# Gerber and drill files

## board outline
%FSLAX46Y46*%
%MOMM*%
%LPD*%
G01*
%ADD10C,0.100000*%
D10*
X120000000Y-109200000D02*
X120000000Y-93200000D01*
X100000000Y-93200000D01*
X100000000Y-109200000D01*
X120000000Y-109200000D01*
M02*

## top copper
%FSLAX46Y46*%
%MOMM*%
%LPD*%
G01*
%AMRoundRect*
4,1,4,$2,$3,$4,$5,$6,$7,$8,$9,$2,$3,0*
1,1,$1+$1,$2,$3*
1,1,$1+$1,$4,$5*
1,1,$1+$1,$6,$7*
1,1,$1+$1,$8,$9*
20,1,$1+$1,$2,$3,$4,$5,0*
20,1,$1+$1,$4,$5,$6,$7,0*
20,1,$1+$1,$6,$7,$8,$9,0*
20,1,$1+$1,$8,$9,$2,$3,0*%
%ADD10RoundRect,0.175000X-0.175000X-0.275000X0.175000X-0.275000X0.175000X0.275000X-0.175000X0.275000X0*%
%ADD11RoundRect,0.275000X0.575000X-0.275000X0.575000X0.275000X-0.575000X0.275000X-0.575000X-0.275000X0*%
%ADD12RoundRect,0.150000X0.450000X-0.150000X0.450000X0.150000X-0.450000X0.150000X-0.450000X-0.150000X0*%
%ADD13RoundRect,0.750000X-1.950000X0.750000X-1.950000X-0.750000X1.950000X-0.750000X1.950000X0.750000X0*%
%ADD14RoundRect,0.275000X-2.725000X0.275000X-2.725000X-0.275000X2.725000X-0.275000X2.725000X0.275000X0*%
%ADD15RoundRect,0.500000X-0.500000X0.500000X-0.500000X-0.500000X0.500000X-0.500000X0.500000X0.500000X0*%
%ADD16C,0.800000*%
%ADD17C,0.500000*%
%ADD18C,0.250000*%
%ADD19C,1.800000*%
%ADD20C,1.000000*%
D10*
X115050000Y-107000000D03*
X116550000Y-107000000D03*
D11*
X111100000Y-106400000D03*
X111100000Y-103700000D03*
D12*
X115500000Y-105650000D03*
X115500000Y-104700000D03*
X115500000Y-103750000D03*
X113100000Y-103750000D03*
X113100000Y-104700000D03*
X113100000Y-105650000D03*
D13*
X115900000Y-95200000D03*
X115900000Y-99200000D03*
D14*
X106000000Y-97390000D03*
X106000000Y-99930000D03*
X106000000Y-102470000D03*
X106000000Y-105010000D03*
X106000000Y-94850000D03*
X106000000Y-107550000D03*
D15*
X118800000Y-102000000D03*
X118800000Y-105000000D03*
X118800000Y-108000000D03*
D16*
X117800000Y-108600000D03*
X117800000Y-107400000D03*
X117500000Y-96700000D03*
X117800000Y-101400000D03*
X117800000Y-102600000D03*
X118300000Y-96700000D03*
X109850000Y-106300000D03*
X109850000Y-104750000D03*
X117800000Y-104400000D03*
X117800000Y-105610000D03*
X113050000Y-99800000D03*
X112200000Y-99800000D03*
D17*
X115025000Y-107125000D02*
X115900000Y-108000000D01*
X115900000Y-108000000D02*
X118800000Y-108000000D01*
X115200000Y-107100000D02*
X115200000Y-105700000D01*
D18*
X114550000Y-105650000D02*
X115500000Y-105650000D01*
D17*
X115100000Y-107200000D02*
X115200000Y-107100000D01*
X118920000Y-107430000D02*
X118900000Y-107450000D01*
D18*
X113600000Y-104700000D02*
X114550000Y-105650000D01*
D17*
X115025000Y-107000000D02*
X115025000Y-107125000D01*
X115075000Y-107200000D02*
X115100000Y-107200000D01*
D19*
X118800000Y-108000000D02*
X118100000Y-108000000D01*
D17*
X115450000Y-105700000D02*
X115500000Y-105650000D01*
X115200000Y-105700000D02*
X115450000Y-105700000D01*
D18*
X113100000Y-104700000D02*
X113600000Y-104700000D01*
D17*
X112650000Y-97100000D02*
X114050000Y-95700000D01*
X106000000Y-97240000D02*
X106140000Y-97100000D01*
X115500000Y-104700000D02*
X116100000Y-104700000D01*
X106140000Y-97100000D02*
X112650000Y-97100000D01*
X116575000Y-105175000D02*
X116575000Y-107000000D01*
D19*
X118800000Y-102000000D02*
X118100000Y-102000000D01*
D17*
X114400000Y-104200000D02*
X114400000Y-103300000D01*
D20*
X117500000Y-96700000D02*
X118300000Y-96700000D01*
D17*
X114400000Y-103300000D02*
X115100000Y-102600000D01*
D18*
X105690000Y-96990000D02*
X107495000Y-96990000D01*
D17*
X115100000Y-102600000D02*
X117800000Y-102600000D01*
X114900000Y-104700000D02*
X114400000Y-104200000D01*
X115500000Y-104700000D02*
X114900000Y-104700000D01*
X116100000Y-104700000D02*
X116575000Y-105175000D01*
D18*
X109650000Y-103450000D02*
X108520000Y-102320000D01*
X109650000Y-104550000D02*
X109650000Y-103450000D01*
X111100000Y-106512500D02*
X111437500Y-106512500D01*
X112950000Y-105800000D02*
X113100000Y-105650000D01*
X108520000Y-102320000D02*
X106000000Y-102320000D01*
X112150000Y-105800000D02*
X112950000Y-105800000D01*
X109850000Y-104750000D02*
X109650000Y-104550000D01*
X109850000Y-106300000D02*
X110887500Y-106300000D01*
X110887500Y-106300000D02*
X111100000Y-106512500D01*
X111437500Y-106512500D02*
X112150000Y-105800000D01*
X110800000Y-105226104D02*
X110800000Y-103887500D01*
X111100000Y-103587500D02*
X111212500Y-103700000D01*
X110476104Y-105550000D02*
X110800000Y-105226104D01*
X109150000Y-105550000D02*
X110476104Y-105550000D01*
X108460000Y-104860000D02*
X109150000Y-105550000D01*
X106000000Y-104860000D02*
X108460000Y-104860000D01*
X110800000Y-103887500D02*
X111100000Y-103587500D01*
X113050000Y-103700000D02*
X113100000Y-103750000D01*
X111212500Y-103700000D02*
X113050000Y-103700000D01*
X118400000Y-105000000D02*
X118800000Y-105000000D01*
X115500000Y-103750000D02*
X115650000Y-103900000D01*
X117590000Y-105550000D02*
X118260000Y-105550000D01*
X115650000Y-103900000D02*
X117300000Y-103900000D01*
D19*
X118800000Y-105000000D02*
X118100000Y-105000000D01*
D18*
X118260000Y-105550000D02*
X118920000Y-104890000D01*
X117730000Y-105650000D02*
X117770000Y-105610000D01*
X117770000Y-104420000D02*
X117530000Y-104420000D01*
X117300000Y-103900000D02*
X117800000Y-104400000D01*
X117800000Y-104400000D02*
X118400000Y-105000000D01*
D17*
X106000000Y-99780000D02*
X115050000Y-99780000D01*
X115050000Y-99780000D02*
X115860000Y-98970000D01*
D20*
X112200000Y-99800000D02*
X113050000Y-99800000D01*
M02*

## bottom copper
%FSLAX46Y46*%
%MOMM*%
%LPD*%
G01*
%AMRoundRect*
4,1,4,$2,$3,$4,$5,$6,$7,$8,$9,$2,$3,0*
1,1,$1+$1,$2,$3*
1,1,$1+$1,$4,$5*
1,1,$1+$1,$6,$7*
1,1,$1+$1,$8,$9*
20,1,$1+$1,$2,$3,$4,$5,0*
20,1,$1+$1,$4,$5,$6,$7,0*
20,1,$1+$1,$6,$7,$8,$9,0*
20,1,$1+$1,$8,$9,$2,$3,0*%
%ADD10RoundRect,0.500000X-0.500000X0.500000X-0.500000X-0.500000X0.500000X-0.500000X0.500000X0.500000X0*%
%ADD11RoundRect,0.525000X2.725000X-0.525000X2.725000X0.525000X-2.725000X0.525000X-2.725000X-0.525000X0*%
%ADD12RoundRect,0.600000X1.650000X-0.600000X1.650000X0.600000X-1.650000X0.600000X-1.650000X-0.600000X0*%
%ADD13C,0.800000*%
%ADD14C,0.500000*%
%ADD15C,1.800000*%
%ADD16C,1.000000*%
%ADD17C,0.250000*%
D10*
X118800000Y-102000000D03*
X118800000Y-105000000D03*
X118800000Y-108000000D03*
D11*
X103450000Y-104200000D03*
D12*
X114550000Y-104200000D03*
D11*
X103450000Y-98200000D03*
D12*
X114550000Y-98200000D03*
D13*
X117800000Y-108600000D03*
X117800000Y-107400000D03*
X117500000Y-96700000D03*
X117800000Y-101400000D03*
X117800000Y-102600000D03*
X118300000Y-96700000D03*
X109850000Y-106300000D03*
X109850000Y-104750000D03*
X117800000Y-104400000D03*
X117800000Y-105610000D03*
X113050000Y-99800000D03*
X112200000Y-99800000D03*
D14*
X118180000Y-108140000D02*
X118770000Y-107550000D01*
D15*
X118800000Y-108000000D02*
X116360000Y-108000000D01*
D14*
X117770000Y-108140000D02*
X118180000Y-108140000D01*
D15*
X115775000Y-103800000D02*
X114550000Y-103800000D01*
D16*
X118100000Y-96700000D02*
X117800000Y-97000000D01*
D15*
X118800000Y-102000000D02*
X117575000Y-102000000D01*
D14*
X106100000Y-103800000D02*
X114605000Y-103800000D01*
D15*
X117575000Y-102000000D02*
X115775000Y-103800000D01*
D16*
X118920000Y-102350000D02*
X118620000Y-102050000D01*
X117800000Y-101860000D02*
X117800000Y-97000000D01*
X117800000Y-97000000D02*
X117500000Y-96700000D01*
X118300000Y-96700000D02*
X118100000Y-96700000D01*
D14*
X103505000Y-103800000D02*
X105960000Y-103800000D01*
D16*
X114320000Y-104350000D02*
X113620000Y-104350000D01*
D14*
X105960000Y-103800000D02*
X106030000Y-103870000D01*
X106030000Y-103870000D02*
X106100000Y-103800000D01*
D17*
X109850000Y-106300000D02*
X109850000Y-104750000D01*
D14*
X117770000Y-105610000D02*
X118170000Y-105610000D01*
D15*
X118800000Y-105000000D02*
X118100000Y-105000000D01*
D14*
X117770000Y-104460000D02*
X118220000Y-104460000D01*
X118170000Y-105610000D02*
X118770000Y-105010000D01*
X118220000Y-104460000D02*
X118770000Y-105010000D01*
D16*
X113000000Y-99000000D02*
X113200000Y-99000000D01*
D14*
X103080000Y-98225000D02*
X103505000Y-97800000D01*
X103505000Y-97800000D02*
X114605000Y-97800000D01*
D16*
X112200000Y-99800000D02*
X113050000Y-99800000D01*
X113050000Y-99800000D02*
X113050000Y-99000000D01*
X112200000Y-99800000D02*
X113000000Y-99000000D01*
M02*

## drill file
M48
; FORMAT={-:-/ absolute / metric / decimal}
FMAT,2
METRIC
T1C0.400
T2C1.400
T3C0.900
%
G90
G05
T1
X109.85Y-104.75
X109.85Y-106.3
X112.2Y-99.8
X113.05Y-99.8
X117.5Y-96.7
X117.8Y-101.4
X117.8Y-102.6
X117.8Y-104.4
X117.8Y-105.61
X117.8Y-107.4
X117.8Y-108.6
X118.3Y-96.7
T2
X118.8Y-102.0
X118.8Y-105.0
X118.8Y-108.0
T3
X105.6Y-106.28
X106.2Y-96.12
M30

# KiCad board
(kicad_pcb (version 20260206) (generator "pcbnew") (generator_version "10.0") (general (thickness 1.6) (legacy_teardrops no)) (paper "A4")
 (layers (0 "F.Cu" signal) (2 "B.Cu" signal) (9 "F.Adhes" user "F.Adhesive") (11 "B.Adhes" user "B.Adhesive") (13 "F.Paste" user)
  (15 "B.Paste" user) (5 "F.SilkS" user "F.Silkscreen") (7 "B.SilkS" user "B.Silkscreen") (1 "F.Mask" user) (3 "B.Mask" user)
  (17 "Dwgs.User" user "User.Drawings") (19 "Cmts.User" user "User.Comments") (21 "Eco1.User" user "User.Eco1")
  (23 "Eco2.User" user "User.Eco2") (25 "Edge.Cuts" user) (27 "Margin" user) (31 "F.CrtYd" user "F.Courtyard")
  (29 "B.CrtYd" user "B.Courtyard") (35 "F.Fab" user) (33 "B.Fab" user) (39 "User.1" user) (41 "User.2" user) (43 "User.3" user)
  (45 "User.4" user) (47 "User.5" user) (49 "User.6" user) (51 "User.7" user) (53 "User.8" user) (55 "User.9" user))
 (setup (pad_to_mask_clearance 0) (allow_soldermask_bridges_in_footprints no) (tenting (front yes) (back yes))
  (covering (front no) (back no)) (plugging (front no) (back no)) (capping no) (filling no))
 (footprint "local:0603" (layer "F.Cu") (at 115.8 107)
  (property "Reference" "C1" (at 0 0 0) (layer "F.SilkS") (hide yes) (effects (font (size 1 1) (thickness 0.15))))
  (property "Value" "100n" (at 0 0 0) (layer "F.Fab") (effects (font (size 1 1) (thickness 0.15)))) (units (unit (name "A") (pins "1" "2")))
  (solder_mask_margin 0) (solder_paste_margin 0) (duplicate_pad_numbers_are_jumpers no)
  (pad "1" smd roundrect (at -0.75 0) (size 0.7 0.9) (layers "F.Cu" "F.Mask" "F.Paste") (roundrect_rratio 0.25) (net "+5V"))
  (pad "2" smd roundrect (at 0.75 0) (size 0.7 0.9) (layers "F.Cu" "F.Mask" "F.Paste") (roundrect_rratio 0.25) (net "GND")))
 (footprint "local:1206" (layer "F.Cu") (at 111.1 105.05 90)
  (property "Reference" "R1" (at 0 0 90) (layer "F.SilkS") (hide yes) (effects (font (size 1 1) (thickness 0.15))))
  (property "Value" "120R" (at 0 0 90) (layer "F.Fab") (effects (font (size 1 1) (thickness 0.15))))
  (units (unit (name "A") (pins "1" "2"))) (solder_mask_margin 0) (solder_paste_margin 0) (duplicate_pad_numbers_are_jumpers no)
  (pad "1" smd roundrect (at -1.35 0 90) (size 1.1 1.7) (layers "F.Cu" "F.Mask" "F.Paste") (roundrect_rratio 0.25) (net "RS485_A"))
  (pad "2" smd roundrect (at 1.35 0 90) (size 1.1 1.7) (layers "F.Cu" "F.Mask" "F.Paste") (roundrect_rratio 0.25) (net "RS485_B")))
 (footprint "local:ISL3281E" (layer "F.Cu") (at 114.3 104.7 90)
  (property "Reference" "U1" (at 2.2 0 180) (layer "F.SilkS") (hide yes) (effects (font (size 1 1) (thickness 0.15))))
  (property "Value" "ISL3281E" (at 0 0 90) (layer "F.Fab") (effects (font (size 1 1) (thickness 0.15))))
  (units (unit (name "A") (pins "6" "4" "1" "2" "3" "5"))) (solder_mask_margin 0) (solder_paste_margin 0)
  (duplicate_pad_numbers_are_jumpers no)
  (pad "1" smd roundrect (at -0.95 1.2 90) (size 0.6 1.2) (layers "F.Cu" "F.Mask" "F.Paste") (roundrect_rratio 0.25) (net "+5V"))
  (pad "2" smd roundrect (at 0 1.2 90) (size 0.6 1.2) (layers "F.Cu" "F.Mask" "F.Paste") (roundrect_rratio 0.25) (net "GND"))
  (pad "3" smd roundrect (at 0.95 1.2 90) (size 0.6 1.2) (layers "F.Cu" "F.Mask" "F.Paste") (roundrect_rratio 0.25) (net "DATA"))
  (pad "4" smd roundrect (at 0.95 -1.2 90) (size 0.6 1.2) (layers "F.Cu" "F.Mask" "F.Paste") (roundrect_rratio 0.25) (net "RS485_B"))
  (pad "5" smd roundrect (at 0 -1.2 90) (size 0.6 1.2) (layers "F.Cu" "F.Mask" "F.Paste") (roundrect_rratio 0.25) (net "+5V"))
  (pad "6" smd roundrect (at -0.95 -1.2 90) (size 0.6 1.2) (layers "F.Cu" "F.Mask" "F.Paste") (roundrect_rratio 0.25) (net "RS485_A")))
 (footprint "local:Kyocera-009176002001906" (layer "F.Cu") (at 115.9 97.2 -90)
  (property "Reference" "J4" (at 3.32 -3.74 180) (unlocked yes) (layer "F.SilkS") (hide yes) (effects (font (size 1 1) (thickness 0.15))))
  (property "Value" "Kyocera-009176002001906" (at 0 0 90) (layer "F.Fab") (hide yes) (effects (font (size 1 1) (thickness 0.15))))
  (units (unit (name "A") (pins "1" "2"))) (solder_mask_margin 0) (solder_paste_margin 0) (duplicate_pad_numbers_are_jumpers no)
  (pad "1" smd roundrect (at -2 0 270) (size 3 5.4) (layers "F.Cu" "F.Mask" "F.Paste") (roundrect_rratio 0.25) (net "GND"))
  (pad "2" smd roundrect (at 2 0 270) (size 3 5.4) (layers "F.Cu" "F.Mask" "F.Paste") (roundrect_rratio 0.25) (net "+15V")))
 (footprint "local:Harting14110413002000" (layer "F.Cu") (at 106 101.2 -90)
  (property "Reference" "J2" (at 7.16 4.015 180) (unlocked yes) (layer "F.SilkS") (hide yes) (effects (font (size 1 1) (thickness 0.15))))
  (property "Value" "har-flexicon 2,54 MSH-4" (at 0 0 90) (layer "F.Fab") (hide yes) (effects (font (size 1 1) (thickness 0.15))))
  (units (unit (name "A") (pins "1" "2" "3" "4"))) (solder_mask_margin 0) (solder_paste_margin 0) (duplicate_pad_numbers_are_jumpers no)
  (pad "" np_thru_hole circle (at -5.08 -0.2 270) (size 0.9 0.9) (drill 0.9) (layers "*.Cu" "*.Mask"))
  (pad "" np_thru_hole circle (at 5.08 0.4 270) (size 0.9 0.9) (drill 0.9) (layers "*.Cu" "*.Mask"))
  (pad "1" smd roundrect (at -3.81 0 270) (size 1.1 6) (layers "F.Cu" "F.Mask" "F.Paste") (roundrect_rratio 0.25) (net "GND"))
  (pad "2" smd roundrect (at -1.27 0 270) (size 1.1 6) (layers "F.Cu" "F.Mask" "F.Paste") (roundrect_rratio 0.25) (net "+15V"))
  (pad "3" smd roundrect (at 1.27 0 270) (size 1.1 6) (layers "F.Cu" "F.Mask" "F.Paste") (roundrect_rratio 0.25) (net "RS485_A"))
  (pad "4" smd roundrect (at 3.81 0 270) (size 1.1 6) (layers "F.Cu" "F.Mask" "F.Paste") (roundrect_rratio 0.25) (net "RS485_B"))
  (pad "MP1" smd roundrect (at -6.35 0 270) (size 1.1 6) (layers "F.Cu" "F.Mask" "F.Paste") (roundrect_rratio 0.25))
  (pad "MP2" smd roundrect (at 6.35 0 270) (size 1.1 6) (layers "F.Cu" "F.Mask" "F.Paste") (roundrect_rratio 0.25)))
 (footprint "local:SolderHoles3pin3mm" (layer "F.Cu") (at 118.8 105 -90)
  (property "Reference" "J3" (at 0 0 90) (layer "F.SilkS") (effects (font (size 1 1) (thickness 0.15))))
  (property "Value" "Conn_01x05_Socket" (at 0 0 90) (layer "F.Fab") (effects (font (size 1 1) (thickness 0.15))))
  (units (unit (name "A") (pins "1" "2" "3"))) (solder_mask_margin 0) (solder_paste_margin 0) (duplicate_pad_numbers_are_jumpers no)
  (pad "1" thru_hole roundrect (at -3 0 270) (size 2 2) (drill 1.4) (layers "*.Cu" "*.Mask") (remove_unused_layers yes)
   (keep_end_layers yes) (zone_layer_connections) (roundrect_rratio 0.25) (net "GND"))
  (pad "2" thru_hole roundrect (at 0 0 270) (size 2 2) (drill 1.4) (layers "*.Cu" "*.Mask") (remove_unused_layers yes) (keep_end_layers yes)
   (zone_layer_connections) (roundrect_rratio 0.25) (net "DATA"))
  (pad "3" thru_hole roundrect (at 3 0 270) (size 2 2) (drill 1.4) (layers "*.Cu" "*.Mask") (remove_unused_layers yes) (keep_end_layers yes)
   (zone_layer_connections) (roundrect_rratio 0.25) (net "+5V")))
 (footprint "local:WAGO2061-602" (layer "B.Cu") (at 108.2 101.2 90)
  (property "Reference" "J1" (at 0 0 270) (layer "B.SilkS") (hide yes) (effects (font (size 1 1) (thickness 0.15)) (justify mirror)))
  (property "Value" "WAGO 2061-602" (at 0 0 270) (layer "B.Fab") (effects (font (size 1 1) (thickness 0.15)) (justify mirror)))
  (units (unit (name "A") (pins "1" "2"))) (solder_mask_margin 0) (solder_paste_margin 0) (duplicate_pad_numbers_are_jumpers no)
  (pad "1" smd roundrect (at -3 -4.75 90) (size 2.1 6.5) (layers "B.Cu" "B.Mask" "B.Paste") (roundrect_rratio 0.25) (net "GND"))
  (pad "1" smd roundrect (at -3 6.35 90) (size 2.4 4.5) (layers "B.Cu" "B.Mask" "B.Paste") (roundrect_rratio 0.25) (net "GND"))
  (pad "2" smd roundrect (at 3 -4.75 90) (size 2.1 6.5) (layers "B.Cu" "B.Mask" "B.Paste") (roundrect_rratio 0.25) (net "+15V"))
  (pad "2" smd roundrect (at 3 6.35 90) (size 2.4 4.5) (layers "B.Cu" "B.Mask" "B.Paste") (roundrect_rratio 0.25) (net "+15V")))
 (gr_poly (pts (xy 120 109.2) (xy 120 93.2) (xy 100 93.2) (xy 100 109.2)) (stroke (width 0.1) (type solid)) (fill no) (layer "Edge.Cuts"))
 (segment (start 115.025 107.125) (end 115.9 108) (width 0.5) (layer "F.Cu") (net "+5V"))
 (segment (start 115.9 108) (end 118.8 108) (width 0.5) (layer "F.Cu") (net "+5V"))
 (segment (start 115.2 107.1) (end 115.2 105.7) (width 0.5) (layer "F.Cu") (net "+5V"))
 (segment (start 114.55 105.65) (end 115.5 105.65) (width 0.25) (layer "F.Cu") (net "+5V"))
 (segment (start 115.1 107.2) (end 115.2 107.1) (width 0.5) (layer "F.Cu") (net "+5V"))
 (segment (start 118.92 107.43) (end 118.9 107.45) (width 0.5) (layer "F.Cu") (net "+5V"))
 (segment (start 113.6 104.7) (end 114.55 105.65) (width 0.25) (layer "F.Cu") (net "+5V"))
 (segment (start 115.025 107) (end 115.025 107.125) (width 0.5) (layer "F.Cu") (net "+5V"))
 (segment (start 115.075 107.2) (end 115.1 107.2) (width 0.5) (layer "F.Cu") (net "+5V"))
 (segment (start 118.8 108) (end 118.1 108) (width 1.8) (layer "F.Cu") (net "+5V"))
 (segment (start 115.45 105.7) (end 115.5 105.65) (width 0.5) (layer "F.Cu") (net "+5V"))
 (segment (start 115.2 105.7) (end 115.45 105.7) (width 0.5) (layer "F.Cu") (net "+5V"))
 (segment (start 113.1 104.7) (end 113.6 104.7) (width 0.25) (layer "F.Cu") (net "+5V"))
 (via (at 117.8 108.6) (size 0.8) (drill 0.4) (layers "F.Cu" "B.Cu") (capping no) (covering (front no) (back no))
  (plugging (front no) (back no)) (filling no) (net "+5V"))
 (via (at 117.8 107.4) (size 0.8) (drill 0.4) (layers "F.Cu" "B.Cu") (capping no) (covering (front no) (back no))
  (plugging (front no) (back no)) (filling no) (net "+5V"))
 (segment (start 118.18 108.14) (end 118.77 107.55) (width 0.5) (layer "B.Cu") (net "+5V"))
 (segment (start 118.8 108) (end 116.36 108) (width 1.8) (layer "B.Cu") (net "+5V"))
 (segment (start 117.77 108.14) (end 118.18 108.14) (width 0.5) (layer "B.Cu") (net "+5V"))
 (segment (start 112.65 97.1) (end 114.05 95.7) (width 0.5) (layer "F.Cu") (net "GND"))
 (segment (start 106 97.24) (end 106.14 97.1) (width 0.5) (layer "F.Cu") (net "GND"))
 (segment (start 115.5 104.7) (end 116.1 104.7) (width 0.5) (layer "F.Cu") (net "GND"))
 (segment (start 106.14 97.1) (end 112.65 97.1) (width 0.5) (layer "F.Cu") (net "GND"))
 (segment (start 116.575 105.175) (end 116.575 107) (width 0.5) (layer "F.Cu") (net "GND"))
 (segment (start 118.8 102) (end 118.1 102) (width 1.8) (layer "F.Cu") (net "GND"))
 (segment (start 114.4 104.2) (end 114.4 103.3) (width 0.5) (layer "F.Cu") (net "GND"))
 (segment (start 117.5 96.7) (end 118.3 96.7) (width 1) (layer "F.Cu") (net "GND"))
 (segment (start 114.4 103.3) (end 115.1 102.6) (width 0.5) (layer "F.Cu") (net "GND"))
 (segment (start 105.69 96.99) (end 107.495 96.99) (width 0.25) (layer "F.Cu") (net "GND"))
 (segment (start 115.1 102.6) (end 117.8 102.6) (width 0.5) (layer "F.Cu") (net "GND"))
 (segment (start 114.9 104.7) (end 114.4 104.2) (width 0.5) (layer "F.Cu") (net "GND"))
 (segment (start 115.5 104.7) (end 114.9 104.7) (width 0.5) (layer "F.Cu") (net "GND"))
 (segment (start 116.1 104.7) (end 116.575 105.175) (width 0.5) (layer "F.Cu") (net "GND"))
 (via (at 117.5 96.7) (size 0.8) (drill 0.4) (layers "F.Cu" "B.Cu") (capping no) (covering (front no) (back no))
  (plugging (front no) (back no)) (filling no) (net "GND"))
 (via (at 117.8 101.4) (size 0.8) (drill 0.4) (layers "F.Cu" "B.Cu") (capping no) (covering (front no) (back no))
  (plugging (front no) (back no)) (filling no) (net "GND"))
 (via (at 117.8 102.6) (size 0.8) (drill 0.4) (layers "F.Cu" "B.Cu") (capping no) (covering (front no) (back no))
  (plugging (front no) (back no)) (filling no) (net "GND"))
 (via (at 118.3 96.7) (size 0.8) (drill 0.4) (layers "F.Cu" "B.Cu") (capping no) (covering (front no) (back no))
  (plugging (front no) (back no)) (filling no) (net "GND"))
 (segment (start 115.775 103.8) (end 114.55 103.8) (width 1.8) (layer "B.Cu") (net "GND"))
 (segment (start 118.1 96.7) (end 117.8 97) (width 1) (layer "B.Cu") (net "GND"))
 (segment (start 118.8 102) (end 117.575 102) (width 1.8) (layer "B.Cu") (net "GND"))
 (segment (start 106.1 103.8) (end 114.605 103.8) (width 0.5) (layer "B.Cu") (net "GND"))
 (segment (start 117.575 102) (end 115.775 103.8) (width 1.8) (layer "B.Cu") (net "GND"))
 (segment (start 118.92 102.35) (end 118.62 102.05) (width 1) (layer "B.Cu") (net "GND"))
 (segment (start 117.8 101.86) (end 117.8 97) (width 1) (layer "B.Cu") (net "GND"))
 (segment (start 117.8 97) (end 117.5 96.7) (width 1) (layer "B.Cu") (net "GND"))
 (segment (start 118.3 96.7) (end 118.1 96.7) (width 1) (layer "B.Cu") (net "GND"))
 (segment (start 103.505 103.8) (end 105.96 103.8) (width 0.5) (layer "B.Cu") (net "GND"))
 (segment (start 114.32 104.35) (end 113.62 104.35) (width 1) (layer "B.Cu") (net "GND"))
 (segment (start 105.96 103.8) (end 106.03 103.87) (width 0.5) (layer "B.Cu") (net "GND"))
 (segment (start 106.03 103.87) (end 106.1 103.8) (width 0.5) (layer "B.Cu") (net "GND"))
 (segment (start 109.65 103.45) (end 108.52 102.32) (width 0.25) (layer "F.Cu") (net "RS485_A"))
 (segment (start 109.65 104.55) (end 109.65 103.45) (width 0.25) (layer "F.Cu") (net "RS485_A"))
 (segment (start 111.1 106.5125) (end 111.4375 106.5125) (width 0.25) (layer "F.Cu") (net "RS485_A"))
 (segment (start 112.95 105.8) (end 113.1 105.65) (width 0.25) (layer "F.Cu") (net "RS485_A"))
 (segment (start 108.52 102.32) (end 106 102.32) (width 0.25) (layer "F.Cu") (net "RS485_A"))
 (segment (start 112.15 105.8) (end 112.95 105.8) (width 0.25) (layer "F.Cu") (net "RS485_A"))
 (segment (start 109.85 104.75) (end 109.65 104.55) (width 0.25) (layer "F.Cu") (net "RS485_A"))
 (segment (start 109.85 106.3) (end 110.8875 106.3) (width 0.25) (layer "F.Cu") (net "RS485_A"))
 (segment (start 110.8875 106.3) (end 111.1 106.5125) (width 0.25) (layer "F.Cu") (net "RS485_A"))
 (segment (start 111.4375 106.5125) (end 112.15 105.8) (width 0.25) (layer "F.Cu") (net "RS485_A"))
 (via (at 109.85 106.3) (size 0.8) (drill 0.4) (layers "F.Cu" "B.Cu") (capping no) (covering (front no) (back no))
  (plugging (front no) (back no)) (filling no) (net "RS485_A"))
 (via (at 109.85 104.75) (size 0.8) (drill 0.4) (layers "F.Cu" "B.Cu") (capping no) (covering (front no) (back no))
  (plugging (front no) (back no)) (filling no) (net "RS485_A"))
 (segment (start 109.85 106.3) (end 109.85 104.75) (width 0.25) (layer "B.Cu") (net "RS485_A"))
 (segment (start 110.8 105.226104) (end 110.8 103.8875) (width 0.25) (layer "F.Cu") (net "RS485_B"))
 (segment (start 111.1 103.5875) (end 111.2125 103.7) (width 0.25) (layer "F.Cu") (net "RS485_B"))
 (segment (start 110.476104 105.55) (end 110.8 105.226104) (width 0.25) (layer "F.Cu") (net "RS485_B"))
 (segment (start 109.15 105.55) (end 110.476104 105.55) (width 0.25) (layer "F.Cu") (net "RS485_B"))
 (segment (start 108.46 104.86) (end 109.15 105.55) (width 0.25) (layer "F.Cu") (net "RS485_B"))
 (segment (start 106 104.86) (end 108.46 104.86) (width 0.25) (layer "F.Cu") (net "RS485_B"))
 (segment (start 110.8 103.8875) (end 111.1 103.5875) (width 0.25) (layer "F.Cu") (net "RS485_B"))
 (segment (start 113.05 103.7) (end 113.1 103.75) (width 0.25) (layer "F.Cu") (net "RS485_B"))
 (segment (start 111.2125 103.7) (end 113.05 103.7) (width 0.25) (layer "F.Cu") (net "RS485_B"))
 (segment (start 118.4 105) (end 118.8 105) (width 0.25) (layer "F.Cu") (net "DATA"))
 (segment (start 115.5 103.75) (end 115.65 103.9) (width 0.25) (layer "F.Cu") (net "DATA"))
 (segment (start 117.59 105.55) (end 118.26 105.55) (width 0.25) (layer "F.Cu") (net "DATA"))
 (segment (start 115.65 103.9) (end 117.3 103.9) (width 0.25) (layer "F.Cu") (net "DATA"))
 (segment (start 118.8 105) (end 118.1 105) (width 1.8) (layer "F.Cu") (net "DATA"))
 (segment (start 118.26 105.55) (end 118.92 104.89) (width 0.25) (layer "F.Cu") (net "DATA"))
 (segment (start 117.73 105.65) (end 117.77 105.61) (width 0.25) (layer "F.Cu") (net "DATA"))
 (segment (start 117.77 104.42) (end 117.53 104.42) (width 0.25) (layer "F.Cu") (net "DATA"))
 (segment (start 117.3 103.9) (end 117.8 104.4) (width 0.25) (layer "F.Cu") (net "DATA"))
 (segment (start 117.8 104.4) (end 118.4 105) (width 0.25) (layer "F.Cu") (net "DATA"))
 (via (at 117.8 104.4) (size 0.8) (drill 0.4) (layers "F.Cu" "B.Cu") (capping no) (covering (front no) (back no))
  (plugging (front no) (back no)) (filling no) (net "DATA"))
 (via (at 117.8 105.61) (size 0.8) (drill 0.4) (layers "F.Cu" "B.Cu") (capping no) (covering (front no) (back no))
  (plugging (front no) (back no)) (filling no) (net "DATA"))
 (segment (start 117.77 105.61) (end 118.17 105.61) (width 0.5) (layer "B.Cu") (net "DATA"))
 (segment (start 118.8 105) (end 118.1 105) (width 1.8) (layer "B.Cu") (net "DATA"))
 (segment (start 117.77 104.46) (end 118.22 104.46) (width 0.5) (layer "B.Cu") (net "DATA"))
 (segment (start 118.17 105.61) (end 118.77 105.01) (width 0.5) (layer "B.Cu") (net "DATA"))
 (segment (start 118.22 104.46) (end 118.77 105.01) (width 0.5) (layer "B.Cu") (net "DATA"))
 (segment (start 106 99.78) (end 115.05 99.78) (width 0.5) (layer "F.Cu") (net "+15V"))
 (segment (start 115.05 99.78) (end 115.86 98.97) (width 0.5) (layer "F.Cu") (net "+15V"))
 (segment (start 112.2 99.8) (end 113.05 99.8) (width 1) (layer "F.Cu") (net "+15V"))
 (via (at 113.05 99.8) (size 0.8) (drill 0.4) (layers "F.Cu" "B.Cu") (capping no) (covering (front no) (back no))
  (plugging (front no) (back no)) (filling no) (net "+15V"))
 (via (at 112.2 99.8) (size 0.8) (drill 0.4) (layers "F.Cu" "B.Cu") (capping no) (covering (front no) (back no))
  (plugging (front no) (back no)) (filling no) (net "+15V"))
 (segment (start 113 99) (end 113.2 99) (width 1) (layer "B.Cu") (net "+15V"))
 (segment (start 103.08 98.225) (end 103.505 97.8) (width 0.5) (layer "B.Cu") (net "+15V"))
 (segment (start 103.505 97.8) (end 114.605 97.8) (width 0.5) (layer "B.Cu") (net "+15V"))
 (segment (start 112.2 99.8) (end 113.05 99.8) (width 1) (layer "B.Cu") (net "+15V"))
 (segment (start 113.05 99.8) (end 113.05 99) (width 1) (layer "B.Cu") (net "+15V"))
 (segment (start 112.2 99.8) (end 113 99) (width 1) (layer "B.Cu") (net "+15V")))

